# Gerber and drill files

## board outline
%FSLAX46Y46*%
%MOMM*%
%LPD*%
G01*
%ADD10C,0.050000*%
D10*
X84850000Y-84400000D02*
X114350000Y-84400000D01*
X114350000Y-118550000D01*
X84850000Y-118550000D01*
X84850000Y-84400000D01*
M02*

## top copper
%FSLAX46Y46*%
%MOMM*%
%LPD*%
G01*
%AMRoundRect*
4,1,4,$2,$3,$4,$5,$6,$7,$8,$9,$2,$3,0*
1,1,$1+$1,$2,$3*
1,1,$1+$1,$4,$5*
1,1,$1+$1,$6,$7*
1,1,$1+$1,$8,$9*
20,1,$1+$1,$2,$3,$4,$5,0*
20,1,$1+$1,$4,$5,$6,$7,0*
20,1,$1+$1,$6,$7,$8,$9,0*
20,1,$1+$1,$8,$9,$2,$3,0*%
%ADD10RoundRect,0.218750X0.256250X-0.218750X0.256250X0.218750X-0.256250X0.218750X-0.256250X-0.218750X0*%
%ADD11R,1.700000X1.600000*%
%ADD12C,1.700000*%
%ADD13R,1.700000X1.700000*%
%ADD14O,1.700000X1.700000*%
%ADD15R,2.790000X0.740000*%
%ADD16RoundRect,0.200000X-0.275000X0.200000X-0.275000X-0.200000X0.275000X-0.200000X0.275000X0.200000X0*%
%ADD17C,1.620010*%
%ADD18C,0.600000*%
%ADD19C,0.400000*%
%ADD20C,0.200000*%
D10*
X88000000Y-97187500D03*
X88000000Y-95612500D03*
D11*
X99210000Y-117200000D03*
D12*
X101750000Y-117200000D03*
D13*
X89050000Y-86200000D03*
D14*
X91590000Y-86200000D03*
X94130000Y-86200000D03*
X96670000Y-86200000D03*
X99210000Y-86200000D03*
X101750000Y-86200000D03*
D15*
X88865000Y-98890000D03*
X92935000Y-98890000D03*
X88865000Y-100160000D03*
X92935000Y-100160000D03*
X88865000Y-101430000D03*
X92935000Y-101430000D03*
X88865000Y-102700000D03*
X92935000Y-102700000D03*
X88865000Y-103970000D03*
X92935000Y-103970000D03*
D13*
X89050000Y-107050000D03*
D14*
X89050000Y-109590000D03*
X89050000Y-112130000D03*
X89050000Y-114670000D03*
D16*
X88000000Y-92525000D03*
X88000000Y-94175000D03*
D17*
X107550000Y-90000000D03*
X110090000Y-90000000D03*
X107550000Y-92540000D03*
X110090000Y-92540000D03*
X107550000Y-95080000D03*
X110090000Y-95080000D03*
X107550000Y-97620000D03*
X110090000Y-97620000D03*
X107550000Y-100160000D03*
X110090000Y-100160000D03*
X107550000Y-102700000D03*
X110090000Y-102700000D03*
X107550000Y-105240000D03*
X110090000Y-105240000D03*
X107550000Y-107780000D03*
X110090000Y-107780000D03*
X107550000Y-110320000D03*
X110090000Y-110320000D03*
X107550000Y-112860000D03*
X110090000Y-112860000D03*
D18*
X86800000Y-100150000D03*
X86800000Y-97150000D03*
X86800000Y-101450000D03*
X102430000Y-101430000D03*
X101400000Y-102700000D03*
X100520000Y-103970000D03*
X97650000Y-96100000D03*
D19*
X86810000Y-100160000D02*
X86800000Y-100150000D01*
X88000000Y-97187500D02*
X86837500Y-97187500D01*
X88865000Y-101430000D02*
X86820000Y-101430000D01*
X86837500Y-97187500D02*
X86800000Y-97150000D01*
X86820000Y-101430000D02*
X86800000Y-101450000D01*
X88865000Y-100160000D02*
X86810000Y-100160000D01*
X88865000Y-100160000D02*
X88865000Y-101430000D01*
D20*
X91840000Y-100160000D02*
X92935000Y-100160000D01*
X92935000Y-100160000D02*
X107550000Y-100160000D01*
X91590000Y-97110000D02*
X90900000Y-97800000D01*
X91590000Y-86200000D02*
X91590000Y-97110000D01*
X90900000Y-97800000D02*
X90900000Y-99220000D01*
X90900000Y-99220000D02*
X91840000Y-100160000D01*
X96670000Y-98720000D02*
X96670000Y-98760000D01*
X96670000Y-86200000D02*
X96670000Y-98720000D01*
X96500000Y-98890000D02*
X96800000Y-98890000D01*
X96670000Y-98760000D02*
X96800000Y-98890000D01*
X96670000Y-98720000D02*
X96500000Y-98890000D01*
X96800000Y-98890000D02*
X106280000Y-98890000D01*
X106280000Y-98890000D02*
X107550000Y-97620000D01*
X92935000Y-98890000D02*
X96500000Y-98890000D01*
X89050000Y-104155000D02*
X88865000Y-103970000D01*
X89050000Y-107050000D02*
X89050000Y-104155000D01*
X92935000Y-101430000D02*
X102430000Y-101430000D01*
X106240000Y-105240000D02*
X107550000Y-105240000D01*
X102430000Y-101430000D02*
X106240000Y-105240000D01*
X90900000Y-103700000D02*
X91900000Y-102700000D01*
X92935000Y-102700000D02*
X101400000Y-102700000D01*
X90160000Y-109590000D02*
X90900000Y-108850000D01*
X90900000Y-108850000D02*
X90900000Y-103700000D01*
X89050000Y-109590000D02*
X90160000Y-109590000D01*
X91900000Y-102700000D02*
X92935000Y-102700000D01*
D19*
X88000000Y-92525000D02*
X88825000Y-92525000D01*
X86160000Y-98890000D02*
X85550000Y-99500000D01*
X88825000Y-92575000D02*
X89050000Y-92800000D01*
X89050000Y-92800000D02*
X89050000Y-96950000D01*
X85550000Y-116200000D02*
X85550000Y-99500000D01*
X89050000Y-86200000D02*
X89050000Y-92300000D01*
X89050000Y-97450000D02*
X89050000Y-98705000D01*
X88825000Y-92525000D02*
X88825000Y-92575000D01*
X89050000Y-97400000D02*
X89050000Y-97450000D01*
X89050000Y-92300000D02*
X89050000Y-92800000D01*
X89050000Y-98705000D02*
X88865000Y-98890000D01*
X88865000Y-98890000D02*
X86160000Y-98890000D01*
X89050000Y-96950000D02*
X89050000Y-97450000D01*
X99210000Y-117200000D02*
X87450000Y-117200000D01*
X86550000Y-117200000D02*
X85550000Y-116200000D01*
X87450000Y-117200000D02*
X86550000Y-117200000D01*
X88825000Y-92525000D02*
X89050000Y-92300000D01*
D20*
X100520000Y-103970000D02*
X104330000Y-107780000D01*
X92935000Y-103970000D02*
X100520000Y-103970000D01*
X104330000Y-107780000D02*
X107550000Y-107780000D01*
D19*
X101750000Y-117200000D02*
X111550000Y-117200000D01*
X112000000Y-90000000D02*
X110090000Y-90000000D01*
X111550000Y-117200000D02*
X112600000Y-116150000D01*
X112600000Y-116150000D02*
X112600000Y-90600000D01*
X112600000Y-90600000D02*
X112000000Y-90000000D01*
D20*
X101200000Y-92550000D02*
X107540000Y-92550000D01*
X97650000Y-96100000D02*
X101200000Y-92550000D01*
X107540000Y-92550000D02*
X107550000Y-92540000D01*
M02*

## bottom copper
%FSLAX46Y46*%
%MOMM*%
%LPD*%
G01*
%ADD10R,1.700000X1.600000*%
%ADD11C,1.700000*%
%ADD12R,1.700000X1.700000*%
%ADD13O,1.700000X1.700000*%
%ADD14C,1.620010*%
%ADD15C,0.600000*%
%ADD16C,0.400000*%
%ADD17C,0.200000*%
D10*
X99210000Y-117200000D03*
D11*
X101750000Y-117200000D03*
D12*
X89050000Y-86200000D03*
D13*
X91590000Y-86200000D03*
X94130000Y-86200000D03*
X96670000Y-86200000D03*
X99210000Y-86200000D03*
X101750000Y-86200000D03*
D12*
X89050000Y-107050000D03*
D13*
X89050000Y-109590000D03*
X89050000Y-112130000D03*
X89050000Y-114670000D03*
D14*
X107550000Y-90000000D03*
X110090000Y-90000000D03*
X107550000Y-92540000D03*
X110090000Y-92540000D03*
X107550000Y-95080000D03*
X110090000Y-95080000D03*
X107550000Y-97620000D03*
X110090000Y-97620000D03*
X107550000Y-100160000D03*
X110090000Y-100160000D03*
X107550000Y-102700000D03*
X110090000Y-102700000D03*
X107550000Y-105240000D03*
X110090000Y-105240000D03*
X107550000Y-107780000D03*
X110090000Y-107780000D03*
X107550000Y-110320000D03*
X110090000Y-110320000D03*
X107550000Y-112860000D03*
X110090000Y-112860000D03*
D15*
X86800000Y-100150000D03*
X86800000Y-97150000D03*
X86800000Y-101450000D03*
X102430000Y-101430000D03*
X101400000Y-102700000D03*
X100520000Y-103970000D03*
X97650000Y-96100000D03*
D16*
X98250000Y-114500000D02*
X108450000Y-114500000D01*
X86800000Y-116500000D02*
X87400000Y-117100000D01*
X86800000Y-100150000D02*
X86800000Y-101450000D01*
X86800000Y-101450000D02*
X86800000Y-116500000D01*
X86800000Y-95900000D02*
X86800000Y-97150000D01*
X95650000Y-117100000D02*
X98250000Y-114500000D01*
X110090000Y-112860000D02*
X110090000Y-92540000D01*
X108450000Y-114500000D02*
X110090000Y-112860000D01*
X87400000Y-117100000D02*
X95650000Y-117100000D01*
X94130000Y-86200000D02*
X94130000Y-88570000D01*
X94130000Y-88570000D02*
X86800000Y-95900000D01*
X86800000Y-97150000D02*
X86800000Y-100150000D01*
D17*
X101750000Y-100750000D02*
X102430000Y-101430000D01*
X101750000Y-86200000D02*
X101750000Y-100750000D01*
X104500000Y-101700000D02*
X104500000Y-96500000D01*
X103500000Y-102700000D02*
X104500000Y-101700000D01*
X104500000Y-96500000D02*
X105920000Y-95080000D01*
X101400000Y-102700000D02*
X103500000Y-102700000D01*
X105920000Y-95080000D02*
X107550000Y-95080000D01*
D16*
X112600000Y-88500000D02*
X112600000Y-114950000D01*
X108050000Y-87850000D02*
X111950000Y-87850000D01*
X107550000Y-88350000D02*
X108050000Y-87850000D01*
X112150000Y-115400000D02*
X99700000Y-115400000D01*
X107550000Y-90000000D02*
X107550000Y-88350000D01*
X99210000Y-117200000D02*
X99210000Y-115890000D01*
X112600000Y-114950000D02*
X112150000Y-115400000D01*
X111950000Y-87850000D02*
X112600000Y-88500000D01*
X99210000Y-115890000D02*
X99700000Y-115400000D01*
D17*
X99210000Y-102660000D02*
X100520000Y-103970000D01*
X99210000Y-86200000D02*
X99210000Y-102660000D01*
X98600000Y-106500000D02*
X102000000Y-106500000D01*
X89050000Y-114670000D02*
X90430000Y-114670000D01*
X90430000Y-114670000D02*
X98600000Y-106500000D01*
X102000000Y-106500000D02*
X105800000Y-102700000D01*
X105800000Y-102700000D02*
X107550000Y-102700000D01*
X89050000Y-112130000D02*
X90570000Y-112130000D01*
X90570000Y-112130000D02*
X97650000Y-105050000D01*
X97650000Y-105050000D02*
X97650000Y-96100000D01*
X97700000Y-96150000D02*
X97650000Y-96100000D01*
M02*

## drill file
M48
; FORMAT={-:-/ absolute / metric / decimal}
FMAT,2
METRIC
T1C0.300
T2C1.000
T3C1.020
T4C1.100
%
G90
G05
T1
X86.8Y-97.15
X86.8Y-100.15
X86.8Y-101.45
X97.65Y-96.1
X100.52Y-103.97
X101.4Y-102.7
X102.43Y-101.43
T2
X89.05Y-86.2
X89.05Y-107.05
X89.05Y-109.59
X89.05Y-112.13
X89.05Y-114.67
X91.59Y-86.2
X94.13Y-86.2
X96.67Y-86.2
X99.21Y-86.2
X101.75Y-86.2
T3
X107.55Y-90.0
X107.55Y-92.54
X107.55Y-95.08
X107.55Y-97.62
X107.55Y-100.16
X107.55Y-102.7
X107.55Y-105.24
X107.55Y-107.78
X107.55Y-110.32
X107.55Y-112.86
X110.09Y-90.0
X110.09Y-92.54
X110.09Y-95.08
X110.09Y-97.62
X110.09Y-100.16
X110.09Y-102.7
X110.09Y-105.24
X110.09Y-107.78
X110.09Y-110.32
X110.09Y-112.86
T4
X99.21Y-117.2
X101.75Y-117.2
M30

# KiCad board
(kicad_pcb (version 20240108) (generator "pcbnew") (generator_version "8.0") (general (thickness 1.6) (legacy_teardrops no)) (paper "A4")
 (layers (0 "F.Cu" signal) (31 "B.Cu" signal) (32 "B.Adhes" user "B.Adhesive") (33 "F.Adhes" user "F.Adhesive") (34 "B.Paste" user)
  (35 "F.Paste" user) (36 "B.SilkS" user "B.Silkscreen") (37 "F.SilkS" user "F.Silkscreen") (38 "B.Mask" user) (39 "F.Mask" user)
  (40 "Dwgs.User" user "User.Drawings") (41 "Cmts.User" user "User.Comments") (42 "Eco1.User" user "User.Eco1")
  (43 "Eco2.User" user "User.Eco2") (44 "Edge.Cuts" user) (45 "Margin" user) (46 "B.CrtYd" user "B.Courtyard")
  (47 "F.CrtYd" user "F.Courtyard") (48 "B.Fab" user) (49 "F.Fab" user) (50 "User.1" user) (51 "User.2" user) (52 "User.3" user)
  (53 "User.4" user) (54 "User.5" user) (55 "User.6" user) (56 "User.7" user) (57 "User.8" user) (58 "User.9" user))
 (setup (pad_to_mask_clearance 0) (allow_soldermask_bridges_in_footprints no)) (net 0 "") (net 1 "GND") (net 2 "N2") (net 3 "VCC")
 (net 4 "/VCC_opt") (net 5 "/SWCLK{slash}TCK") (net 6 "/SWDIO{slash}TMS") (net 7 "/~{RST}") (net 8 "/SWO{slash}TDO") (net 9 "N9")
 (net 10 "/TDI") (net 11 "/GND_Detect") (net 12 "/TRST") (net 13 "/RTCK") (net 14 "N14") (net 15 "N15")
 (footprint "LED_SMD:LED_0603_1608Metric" (layer "F.Cu") (at 88 96.4 90)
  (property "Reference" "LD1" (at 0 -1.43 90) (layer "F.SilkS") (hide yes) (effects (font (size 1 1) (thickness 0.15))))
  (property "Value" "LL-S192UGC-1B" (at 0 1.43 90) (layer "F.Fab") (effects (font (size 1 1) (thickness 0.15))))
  (pad "1" smd roundrect (at -0.7875 0 90) (size 0.875 0.95) (layers "F.Cu" "F.Paste" "F.Mask") (roundrect_rratio 0.25) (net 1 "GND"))
  (pad "2" smd roundrect (at 0.7875 0 90) (size 0.875 0.95) (layers "F.Cu" "F.Paste" "F.Mask") (roundrect_rratio 0.25) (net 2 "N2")))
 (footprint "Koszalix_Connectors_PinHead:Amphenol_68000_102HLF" (layer "F.Cu") (at 100.71 117.2)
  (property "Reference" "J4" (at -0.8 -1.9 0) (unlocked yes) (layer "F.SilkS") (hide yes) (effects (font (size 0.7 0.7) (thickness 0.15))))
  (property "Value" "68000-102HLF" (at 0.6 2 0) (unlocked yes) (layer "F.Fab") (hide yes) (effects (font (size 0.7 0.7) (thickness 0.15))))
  (pad "1" thru_hole rect (at -1.5 0) (size 1.7 1.6) (drill 1.1) (layers "*.Cu" "*.Mask") (remove_unused_layers no) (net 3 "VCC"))
  (pad "2" thru_hole circle (at 1.04 0) (size 1.7 1.7) (drill 1.1) (layers "*.Cu" "*.Mask") (remove_unused_layers no) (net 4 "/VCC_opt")))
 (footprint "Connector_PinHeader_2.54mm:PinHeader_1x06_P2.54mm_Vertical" (layer "F.Cu") (at 89.05 86.2 90)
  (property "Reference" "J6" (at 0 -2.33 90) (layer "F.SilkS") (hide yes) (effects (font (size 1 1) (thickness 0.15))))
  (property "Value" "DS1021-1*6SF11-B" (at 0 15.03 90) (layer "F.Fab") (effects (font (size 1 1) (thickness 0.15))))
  (pad "1" thru_hole rect (at 0 0 90) (size 1.7 1.7) (drill 1) (layers "*.Cu" "*.Mask") (remove_unused_layers no) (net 3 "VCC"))
  (pad "2" thru_hole oval (at 0 2.54 90) (size 1.7 1.7) (drill 1) (layers "*.Cu" "*.Mask") (remove_unused_layers no)
   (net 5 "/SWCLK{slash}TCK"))
  (pad "3" thru_hole oval (at 0 5.08 90) (size 1.7 1.7) (drill 1) (layers "*.Cu" "*.Mask") (remove_unused_layers no) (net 1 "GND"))
  (pad "4" thru_hole oval (at 0 7.62 90) (size 1.7 1.7) (drill 1) (layers "*.Cu" "*.Mask") (remove_unused_layers no)
   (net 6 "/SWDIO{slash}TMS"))
  (pad "5" thru_hole oval (at 0 10.16 90) (size 1.7 1.7) (drill 1) (layers "*.Cu" "*.Mask") (remove_unused_layers no) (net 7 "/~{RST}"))
  (pad "6" thru_hole oval (at 0 12.7 90) (size 1.7 1.7) (drill 1) (layers "*.Cu" "*.Mask") (remove_unused_layers no)
   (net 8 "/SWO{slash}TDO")))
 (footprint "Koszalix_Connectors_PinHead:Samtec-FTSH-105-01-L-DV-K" (layer "F.Cu") (at 90.9 101.43 -90)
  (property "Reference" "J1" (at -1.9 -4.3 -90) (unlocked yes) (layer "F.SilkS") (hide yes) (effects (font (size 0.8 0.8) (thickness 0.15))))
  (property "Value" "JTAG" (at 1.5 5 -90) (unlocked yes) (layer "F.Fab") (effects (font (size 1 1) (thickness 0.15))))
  (pad "1" smd rect (at -2.54 2.035 270) (size 0.74 2.79) (layers "F.Cu" "F.Paste" "F.Mask") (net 3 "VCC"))
  (pad "2" smd rect (at -2.54 -2.035 270) (size 0.74 2.79) (layers "F.Cu" "F.Paste" "F.Mask") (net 6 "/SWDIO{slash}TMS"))
  (pad "3" smd rect (at -1.27 2.035 270) (size 0.74 2.79) (layers "F.Cu" "F.Paste" "F.Mask") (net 1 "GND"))
  (pad "4" smd rect (at -1.27 -2.035 270) (size 0.74 2.79) (layers "F.Cu" "F.Paste" "F.Mask") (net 5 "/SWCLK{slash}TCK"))
  (pad "5" smd rect (at 0 2.035 270) (size 0.74 2.79) (layers "F.Cu" "F.Paste" "F.Mask") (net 1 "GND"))
  (pad "6" smd rect (at 0 -2.035 270) (size 0.74 2.79) (layers "F.Cu" "F.Paste" "F.Mask") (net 8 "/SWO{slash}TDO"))
  (pad "7" smd rect (at 1.27 2.035 270) (size 0.74 2.79) (layers "F.Cu" "F.Paste" "F.Mask") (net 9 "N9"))
  (pad "8" smd rect (at 1.27 -2.035 270) (size 0.74 2.79) (layers "F.Cu" "F.Paste" "F.Mask") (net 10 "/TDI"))
  (pad "9" smd rect (at 2.54 2.035 270) (size 0.74 2.79) (layers "F.Cu" "F.Paste" "F.Mask") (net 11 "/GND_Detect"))
  (pad "10" smd rect (at 2.54 -2.035 270) (size 0.74 2.79) (layers "F.Cu" "F.Paste" "F.Mask") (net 7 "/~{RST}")))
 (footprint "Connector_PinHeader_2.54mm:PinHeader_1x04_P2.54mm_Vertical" (layer "F.Cu") (at 89.05 107.05)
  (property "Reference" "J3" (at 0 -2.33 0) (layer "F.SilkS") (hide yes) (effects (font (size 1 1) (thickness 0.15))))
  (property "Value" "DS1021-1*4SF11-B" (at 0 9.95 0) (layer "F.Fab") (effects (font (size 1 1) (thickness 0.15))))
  (pad "1" thru_hole rect (at 0 0) (size 1.7 1.7) (drill 1) (layers "*.Cu" "*.Mask") (remove_unused_layers no) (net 11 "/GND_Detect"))
  (pad "2" thru_hole oval (at 0 2.54) (size 1.7 1.7) (drill 1) (layers "*.Cu" "*.Mask") (remove_unused_layers no) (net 10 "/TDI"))
  (pad "3" thru_hole oval (at 0 5.08) (size 1.7 1.7) (drill 1) (layers "*.Cu" "*.Mask") (remove_unused_layers no) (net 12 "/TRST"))
  (pad "4" thru_hole oval (at 0 7.62) (size 1.7 1.7) (drill 1) (layers "*.Cu" "*.Mask") (remove_unused_layers no) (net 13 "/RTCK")))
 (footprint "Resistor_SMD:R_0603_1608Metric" (layer "F.Cu") (at 88 93.35 -90)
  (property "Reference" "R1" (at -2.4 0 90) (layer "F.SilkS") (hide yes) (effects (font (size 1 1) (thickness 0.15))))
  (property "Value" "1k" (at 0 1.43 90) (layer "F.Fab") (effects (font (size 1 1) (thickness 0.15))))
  (pad "1" smd roundrect (at -0.825 0 270) (size 0.8 0.95) (layers "F.Cu" "F.Paste" "F.Mask") (roundrect_rratio 0.25) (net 3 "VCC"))
  (pad "2" smd roundrect (at 0.825 0 270) (size 0.8 0.95) (layers "F.Cu" "F.Paste" "F.Mask") (roundrect_rratio 0.25) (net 2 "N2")))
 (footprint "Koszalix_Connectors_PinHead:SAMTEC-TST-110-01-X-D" (layer "F.Cu") (at 109.00999 101.43 -90)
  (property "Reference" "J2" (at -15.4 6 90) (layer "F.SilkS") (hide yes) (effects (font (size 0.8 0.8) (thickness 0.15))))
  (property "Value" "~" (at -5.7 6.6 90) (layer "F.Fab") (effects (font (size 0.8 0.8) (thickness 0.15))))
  (pad "1" thru_hole circle (at -11.43 1.45999 270) (size 1.62001 1.62001) (drill 1.01999) (layers "*.Cu") (remove_unused_layers no)
   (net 3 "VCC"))
  (pad "2" thru_hole circle (at -11.43 -1.08001 270) (size 1.62001 1.62001) (drill 1.01999) (layers "*.Cu") (remove_unused_layers no)
   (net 4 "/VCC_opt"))
  (pad "3" thru_hole circle (at -8.89 1.45999 270) (size 1.62001 1.62001) (drill 1.01999) (layers "*.Cu") (remove_unused_layers no)
   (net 12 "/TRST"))
  (pad "4" thru_hole circle (at -8.89 -1.08001 270) (size 1.62001 1.62001) (drill 1.01999) (layers "*.Cu") (remove_unused_layers no)
   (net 1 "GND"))
  (pad "5" thru_hole circle (at -6.35 1.45999 270) (size 1.62001 1.62001) (drill 1.01999) (layers "*.Cu") (remove_unused_layers no)
   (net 10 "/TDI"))
  (pad "6" thru_hole circle (at -6.35 -1.08001 270) (size 1.62001 1.62001) (drill 1.01999) (layers "*.Cu") (remove_unused_layers no)
   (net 1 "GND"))
  (pad "7" thru_hole circle (at -3.81 1.45999 270) (size 1.62001 1.62001) (drill 1.01999) (layers "*.Cu") (remove_unused_layers no)
   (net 6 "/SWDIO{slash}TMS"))
  (pad "8" thru_hole circle (at -3.81 -1.08001 270) (size 1.62001 1.62001) (drill 1.01999) (layers "*.Cu") (remove_unused_layers no)
   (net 1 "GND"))
  (pad "9" thru_hole circle (at -1.27 1.45999 270) (size 1.62001 1.62001) (drill 1.01999) (layers "*.Cu") (remove_unused_layers no)
   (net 5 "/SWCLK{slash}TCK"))
  (pad "10" thru_hole circle (at -1.27 -1.08001 270) (size 1.62001 1.62001) (drill 1.01999) (layers "*.Cu") (remove_unused_layers no)
   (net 1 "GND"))
  (pad "11" thru_hole circle (at 1.27 1.45999 270) (size 1.62001 1.62001) (drill 1.01999) (layers "*.Cu") (remove_unused_layers no)
   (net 13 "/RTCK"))
  (pad "12" thru_hole circle (at 1.27 -1.08001 270) (size 1.62001 1.62001) (drill 1.01999) (layers "*.Cu") (remove_unused_layers no)
   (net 1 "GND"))
  (pad "13" thru_hole circle (at 3.81 1.45999 270) (size 1.62001 1.62001) (drill 1.01999) (layers "*.Cu") (remove_unused_layers no)
   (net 8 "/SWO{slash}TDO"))
  (pad "14" thru_hole circle (at 3.81 -1.08001 270) (size 1.62001 1.62001) (drill 1.01999) (layers "*.Cu") (remove_unused_layers no)
   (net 1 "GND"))
  (pad "15" thru_hole circle (at 6.35 1.45999 270) (size 1.62001 1.62001) (drill 1.01999) (layers "*.Cu") (remove_unused_layers no)
   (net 7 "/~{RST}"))
  (pad "16" thru_hole circle (at 6.35 -1.08001 270) (size 1.62001 1.62001) (drill 1.01999) (layers "*.Cu") (remove_unused_layers no)
   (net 1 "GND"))
  (pad "17" thru_hole circle (at 8.89 1.45999 270) (size 1.62001 1.62001) (drill 1.01999) (layers "*.Cu") (remove_unused_layers no)
   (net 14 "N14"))
  (pad "18" thru_hole circle (at 8.89 -1.08001 270) (size 1.62001 1.62001) (drill 1.01999) (layers "*.Cu") (remove_unused_layers no)
   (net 1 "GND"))
  (pad "19" thru_hole circle (at 11.43 1.45999 270) (size 1.62001 1.62001) (drill 1.01999) (layers "*.Cu") (remove_unused_layers no)
   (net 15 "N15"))
  (pad "20" thru_hole circle (at 11.43 -1.08001 270) (size 1.62001 1.62001) (drill 1.01999) (layers "*.Cu") (remove_unused_layers no)
   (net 1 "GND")))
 (gr_rect (start 84.85 84.4) (end 114.35 118.55) (stroke (width 0.05) (type default)) (fill none) (layer "Edge.Cuts"))
 (segment (start 86.81 100.16) (end 86.8 100.15) (width 0.4) (layer "F.Cu") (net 1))
 (segment (start 88 97.1875) (end 86.8375 97.1875) (width 0.4) (layer "F.Cu") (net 1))
 (segment (start 88.865 101.43) (end 86.82 101.43) (width 0.4) (layer "F.Cu") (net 1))
 (segment (start 86.8375 97.1875) (end 86.8 97.15) (width 0.4) (layer "F.Cu") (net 1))
 (segment (start 86.82 101.43) (end 86.8 101.45) (width 0.4) (layer "F.Cu") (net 1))
 (segment (start 88.865 100.16) (end 86.81 100.16) (width 0.4) (layer "F.Cu") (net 1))
 (segment (start 88.865 100.16) (end 88.865 101.43) (width 0.4) (layer "F.Cu") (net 1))
 (via (at 86.8 100.15) (size 0.6) (drill 0.3) (layers "F.Cu" "B.Cu") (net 1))
 (via (at 86.8 97.15) (size 0.6) (drill 0.3) (layers "F.Cu" "B.Cu") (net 1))
 (via (at 86.8 101.45) (size 0.6) (drill 0.3) (layers "F.Cu" "B.Cu") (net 1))
 (segment (start 98.25 114.5) (end 108.45 114.5) (width 0.4) (layer "B.Cu") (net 1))
 (segment (start 86.8 116.5) (end 87.4 117.1) (width 0.4) (layer "B.Cu") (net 1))
 (segment (start 86.8 100.15) (end 86.8 101.45) (width 0.4) (layer "B.Cu") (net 1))
 (segment (start 86.8 101.45) (end 86.8 116.5) (width 0.4) (layer "B.Cu") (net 1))
 (segment (start 86.8 95.9) (end 86.8 97.15) (width 0.4) (layer "B.Cu") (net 1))
 (segment (start 95.65 117.1) (end 98.25 114.5) (width 0.4) (layer "B.Cu") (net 1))
 (segment (start 110.09 112.86) (end 110.09 92.54) (width 0.4) (layer "B.Cu") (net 1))
 (segment (start 108.45 114.5) (end 110.09 112.86) (width 0.4) (layer "B.Cu") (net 1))
 (segment (start 87.4 117.1) (end 95.65 117.1) (width 0.4) (layer "B.Cu") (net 1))
 (segment (start 94.13 86.2) (end 94.13 88.57) (width 0.4) (layer "B.Cu") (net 1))
 (segment (start 94.13 88.57) (end 86.8 95.9) (width 0.4) (layer "B.Cu") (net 1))
 (segment (start 86.8 97.15) (end 86.8 100.15) (width 0.4) (layer "B.Cu") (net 1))
 (segment (start 91.84 100.16) (end 92.935 100.16) (width 0.2) (layer "F.Cu") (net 5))
 (segment (start 92.935 100.16) (end 107.55 100.16) (width 0.2) (layer "F.Cu") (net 5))
 (segment (start 91.59 97.11) (end 90.9 97.8) (width 0.2) (layer "F.Cu") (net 5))
 (segment (start 91.59 86.2) (end 91.59 97.11) (width 0.2) (layer "F.Cu") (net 5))
 (segment (start 90.9 97.8) (end 90.9 99.22) (width 0.2) (layer "F.Cu") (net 5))
 (segment (start 90.9 99.22) (end 91.84 100.16) (width 0.2) (layer "F.Cu") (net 5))
 (segment (start 96.67 98.72) (end 96.67 98.76) (width 0.2) (layer "F.Cu") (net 6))
 (segment (start 96.67 86.2) (end 96.67 98.72) (width 0.2) (layer "F.Cu") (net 6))
 (segment (start 96.5 98.89) (end 96.8 98.89) (width 0.2) (layer "F.Cu") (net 6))
 (segment (start 96.67 98.76) (end 96.8 98.89) (width 0.2) (layer "F.Cu") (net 6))
 (segment (start 96.67 98.72) (end 96.5 98.89) (width 0.2) (layer "F.Cu") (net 6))
 (segment (start 96.8 98.89) (end 106.28 98.89) (width 0.2) (layer "F.Cu") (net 6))
 (segment (start 106.28 98.89) (end 107.55 97.62) (width 0.2) (layer "F.Cu") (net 6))
 (segment (start 92.935 98.89) (end 96.5 98.89) (width 0.2) (layer "F.Cu") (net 6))
 (segment (start 89.05 104.155) (end 88.865 103.97) (width 0.2) (layer "F.Cu") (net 11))
 (segment (start 89.05 107.05) (end 89.05 104.155) (width 0.2) (layer "F.Cu") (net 11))
 (segment (start 92.935 101.43) (end 102.43 101.43) (width 0.2) (layer "F.Cu") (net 8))
 (segment (start 106.24 105.24) (end 107.55 105.24) (width 0.2) (layer "F.Cu") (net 8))
 (segment (start 102.43 101.43) (end 106.24 105.24) (width 0.2) (layer "F.Cu") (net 8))
 (via (at 102.43 101.43) (size 0.6) (drill 0.3) (layers "F.Cu" "B.Cu") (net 8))
 (segment (start 101.75 100.75) (end 102.43 101.43) (width 0.2) (layer "B.Cu") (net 8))
 (segment (start 101.75 86.2) (end 101.75 100.75) (width 0.2) (layer "B.Cu") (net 8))
 (segment (start 90.9 103.7) (end 91.9 102.7) (width 0.2) (layer "F.Cu") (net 10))
 (segment (start 92.935 102.7) (end 101.4 102.7) (width 0.2) (layer "F.Cu") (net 10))
 (segment (start 90.16 109.59) (end 90.9 108.85) (width 0.2) (layer "F.Cu") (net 10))
 (segment (start 90.9 108.85) (end 90.9 103.7) (width 0.2) (layer "F.Cu") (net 10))
 (segment (start 89.05 109.59) (end 90.16 109.59) (width 0.2) (layer "F.Cu") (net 10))
 (segment (start 91.9 102.7) (end 92.935 102.7) (width 0.2) (layer "F.Cu") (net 10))
 (via (at 101.4 102.7) (size 0.6) (drill 0.3) (layers "F.Cu" "B.Cu") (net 10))
 (segment (start 104.5 101.7) (end 104.5 96.5) (width 0.2) (layer "B.Cu") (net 10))
 (segment (start 103.5 102.7) (end 104.5 101.7) (width 0.2) (layer "B.Cu") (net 10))
 (segment (start 104.5 96.5) (end 105.92 95.08) (width 0.2) (layer "B.Cu") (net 10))
 (segment (start 101.4 102.7) (end 103.5 102.7) (width 0.2) (layer "B.Cu") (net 10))
 (segment (start 105.92 95.08) (end 107.55 95.08) (width 0.2) (layer "B.Cu") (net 10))
 (segment (start 88 92.525) (end 88.825 92.525) (width 0.4) (layer "F.Cu") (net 3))
 (segment (start 86.16 98.89) (end 85.55 99.5) (width 0.4) (layer "F.Cu") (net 3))
 (segment (start 88.825 92.575) (end 89.05 92.8) (width 0.4) (layer "F.Cu") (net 3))
 (segment (start 89.05 92.8) (end 89.05 96.95) (width 0.4) (layer "F.Cu") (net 3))
 (segment (start 85.55 116.2) (end 85.55 99.5) (width 0.4) (layer "F.Cu") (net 3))
 (segment (start 89.05 86.2) (end 89.05 92.3) (width 0.4) (layer "F.Cu") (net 3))
 (segment (start 89.05 97.45) (end 89.05 98.705) (width 0.4) (layer "F.Cu") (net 3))
 (segment (start 88.825 92.525) (end 88.825 92.575) (width 0.4) (layer "F.Cu") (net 3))
 (segment (start 89.05 97.4) (end 89.05 97.45) (width 0.4) (layer "F.Cu") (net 3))
 (segment (start 89.05 92.3) (end 89.05 92.8) (width 0.4) (layer "F.Cu") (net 3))
 (segment (start 89.05 98.705) (end 88.865 98.89) (width 0.4) (layer "F.Cu") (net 3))
 (segment (start 88.865 98.89) (end 86.16 98.89) (width 0.4) (layer "F.Cu") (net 3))
 (segment (start 89.05 96.95) (end 89.05 97.45) (width 0.4) (layer "F.Cu") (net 3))
 (segment (start 99.21 117.2) (end 87.45 117.2) (width 0.4) (layer "F.Cu") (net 3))
 (segment (start 86.55 117.2) (end 85.55 116.2) (width 0.4) (layer "F.Cu") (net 3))
 (segment (start 87.45 117.2) (end 86.55 117.2) (width 0.4) (layer "F.Cu") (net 3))
 (segment (start 88.825 92.525) (end 89.05 92.3) (width 0.4) (layer "F.Cu") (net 3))
 (segment (start 112.6 88.5) (end 112.6 114.95) (width 0.4) (layer "B.Cu") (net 3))
 (segment (start 108.05 87.85) (end 111.95 87.85) (width 0.4) (layer "B.Cu") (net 3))
 (segment (start 107.55 88.35) (end 108.05 87.85) (width 0.4) (layer "B.Cu") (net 3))
 (segment (start 112.15 115.4) (end 99.7 115.4) (width 0.4) (layer "B.Cu") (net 3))
 (segment (start 107.55 90) (end 107.55 88.35) (width 0.4) (layer "B.Cu") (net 3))
 (segment (start 99.21 117.2) (end 99.21 115.89) (width 0.4) (layer "B.Cu") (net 3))
 (segment (start 112.6 114.95) (end 112.15 115.4) (width 0.4) (layer "B.Cu") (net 3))
 (segment (start 111.95 87.85) (end 112.6 88.5) (width 0.4) (layer "B.Cu") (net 3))
 (segment (start 99.21 115.89) (end 99.7 115.4) (width 0.4) (layer "B.Cu") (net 3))
 (segment (start 100.52 103.97) (end 104.33 107.78) (width 0.2) (layer "F.Cu") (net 7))
 (segment (start 92.935 103.97) (end 100.52 103.97) (width 0.2) (layer "F.Cu") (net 7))
 (segment (start 104.33 107.78) (end 107.55 107.78) (width 0.2) (layer "F.Cu") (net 7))
 (via (at 100.52 103.97) (size 0.6) (drill 0.3) (layers "F.Cu" "B.Cu") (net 7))
 (segment (start 99.21 102.66) (end 100.52 103.97) (width 0.2) (layer "B.Cu") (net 7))
 (segment (start 99.21 86.2) (end 99.21 102.66) (width 0.2) (layer "B.Cu") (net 7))
 (segment (start 101.75 117.2) (end 111.55 117.2) (width 0.4) (layer "F.Cu") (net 4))
 (segment (start 112 90) (end 110.09 90) (width 0.4) (layer "F.Cu") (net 4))
 (segment (start 111.55 117.2) (end 112.6 116.15) (width 0.4) (layer "F.Cu") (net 4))
 (segment (start 112.6 116.15) (end 112.6 90.6) (width 0.4) (layer "F.Cu") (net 4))
 (segment (start 112.6 90.6) (end 112 90) (width 0.4) (layer "F.Cu") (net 4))
 (segment (start 98.6 106.5) (end 102 106.5) (width 0.2) (layer "B.Cu") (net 13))
 (segment (start 89.05 114.67) (end 90.43 114.67) (width 0.2) (layer "B.Cu") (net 13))
 (segment (start 90.43 114.67) (end 98.6 106.5) (width 0.2) (layer "B.Cu") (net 13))
 (segment (start 102 106.5) (end 105.8 102.7) (width 0.2) (layer "B.Cu") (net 13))
 (segment (start 105.8 102.7) (end 107.55 102.7) (width 0.2) (layer "B.Cu") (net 13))
 (segment (start 101.2 92.55) (end 107.54 92.55) (width 0.2) (layer "F.Cu") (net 12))
 (segment (start 97.65 96.1) (end 101.2 92.55) (width 0.2) (layer "F.Cu") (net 12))
 (segment (start 107.54 92.55) (end 107.55 92.54) (width 0.2) (layer "F.Cu") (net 12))
 (via (at 97.65 96.1) (size 0.6) (drill 0.3) (layers "F.Cu" "B.Cu") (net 12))
 (segment (start 89.05 112.13) (end 90.57 112.13) (width 0.2) (layer "B.Cu") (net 12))
 (segment (start 90.57 112.13) (end 97.65 105.05) (width 0.2) (layer "B.Cu") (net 12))
 (segment (start 97.65 105.05) (end 97.65 96.1) (width 0.2) (layer "B.Cu") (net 12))
 (segment (start 97.7 96.15) (end 97.65 96.1) (width 0.2) (layer "B.Cu") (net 12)))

